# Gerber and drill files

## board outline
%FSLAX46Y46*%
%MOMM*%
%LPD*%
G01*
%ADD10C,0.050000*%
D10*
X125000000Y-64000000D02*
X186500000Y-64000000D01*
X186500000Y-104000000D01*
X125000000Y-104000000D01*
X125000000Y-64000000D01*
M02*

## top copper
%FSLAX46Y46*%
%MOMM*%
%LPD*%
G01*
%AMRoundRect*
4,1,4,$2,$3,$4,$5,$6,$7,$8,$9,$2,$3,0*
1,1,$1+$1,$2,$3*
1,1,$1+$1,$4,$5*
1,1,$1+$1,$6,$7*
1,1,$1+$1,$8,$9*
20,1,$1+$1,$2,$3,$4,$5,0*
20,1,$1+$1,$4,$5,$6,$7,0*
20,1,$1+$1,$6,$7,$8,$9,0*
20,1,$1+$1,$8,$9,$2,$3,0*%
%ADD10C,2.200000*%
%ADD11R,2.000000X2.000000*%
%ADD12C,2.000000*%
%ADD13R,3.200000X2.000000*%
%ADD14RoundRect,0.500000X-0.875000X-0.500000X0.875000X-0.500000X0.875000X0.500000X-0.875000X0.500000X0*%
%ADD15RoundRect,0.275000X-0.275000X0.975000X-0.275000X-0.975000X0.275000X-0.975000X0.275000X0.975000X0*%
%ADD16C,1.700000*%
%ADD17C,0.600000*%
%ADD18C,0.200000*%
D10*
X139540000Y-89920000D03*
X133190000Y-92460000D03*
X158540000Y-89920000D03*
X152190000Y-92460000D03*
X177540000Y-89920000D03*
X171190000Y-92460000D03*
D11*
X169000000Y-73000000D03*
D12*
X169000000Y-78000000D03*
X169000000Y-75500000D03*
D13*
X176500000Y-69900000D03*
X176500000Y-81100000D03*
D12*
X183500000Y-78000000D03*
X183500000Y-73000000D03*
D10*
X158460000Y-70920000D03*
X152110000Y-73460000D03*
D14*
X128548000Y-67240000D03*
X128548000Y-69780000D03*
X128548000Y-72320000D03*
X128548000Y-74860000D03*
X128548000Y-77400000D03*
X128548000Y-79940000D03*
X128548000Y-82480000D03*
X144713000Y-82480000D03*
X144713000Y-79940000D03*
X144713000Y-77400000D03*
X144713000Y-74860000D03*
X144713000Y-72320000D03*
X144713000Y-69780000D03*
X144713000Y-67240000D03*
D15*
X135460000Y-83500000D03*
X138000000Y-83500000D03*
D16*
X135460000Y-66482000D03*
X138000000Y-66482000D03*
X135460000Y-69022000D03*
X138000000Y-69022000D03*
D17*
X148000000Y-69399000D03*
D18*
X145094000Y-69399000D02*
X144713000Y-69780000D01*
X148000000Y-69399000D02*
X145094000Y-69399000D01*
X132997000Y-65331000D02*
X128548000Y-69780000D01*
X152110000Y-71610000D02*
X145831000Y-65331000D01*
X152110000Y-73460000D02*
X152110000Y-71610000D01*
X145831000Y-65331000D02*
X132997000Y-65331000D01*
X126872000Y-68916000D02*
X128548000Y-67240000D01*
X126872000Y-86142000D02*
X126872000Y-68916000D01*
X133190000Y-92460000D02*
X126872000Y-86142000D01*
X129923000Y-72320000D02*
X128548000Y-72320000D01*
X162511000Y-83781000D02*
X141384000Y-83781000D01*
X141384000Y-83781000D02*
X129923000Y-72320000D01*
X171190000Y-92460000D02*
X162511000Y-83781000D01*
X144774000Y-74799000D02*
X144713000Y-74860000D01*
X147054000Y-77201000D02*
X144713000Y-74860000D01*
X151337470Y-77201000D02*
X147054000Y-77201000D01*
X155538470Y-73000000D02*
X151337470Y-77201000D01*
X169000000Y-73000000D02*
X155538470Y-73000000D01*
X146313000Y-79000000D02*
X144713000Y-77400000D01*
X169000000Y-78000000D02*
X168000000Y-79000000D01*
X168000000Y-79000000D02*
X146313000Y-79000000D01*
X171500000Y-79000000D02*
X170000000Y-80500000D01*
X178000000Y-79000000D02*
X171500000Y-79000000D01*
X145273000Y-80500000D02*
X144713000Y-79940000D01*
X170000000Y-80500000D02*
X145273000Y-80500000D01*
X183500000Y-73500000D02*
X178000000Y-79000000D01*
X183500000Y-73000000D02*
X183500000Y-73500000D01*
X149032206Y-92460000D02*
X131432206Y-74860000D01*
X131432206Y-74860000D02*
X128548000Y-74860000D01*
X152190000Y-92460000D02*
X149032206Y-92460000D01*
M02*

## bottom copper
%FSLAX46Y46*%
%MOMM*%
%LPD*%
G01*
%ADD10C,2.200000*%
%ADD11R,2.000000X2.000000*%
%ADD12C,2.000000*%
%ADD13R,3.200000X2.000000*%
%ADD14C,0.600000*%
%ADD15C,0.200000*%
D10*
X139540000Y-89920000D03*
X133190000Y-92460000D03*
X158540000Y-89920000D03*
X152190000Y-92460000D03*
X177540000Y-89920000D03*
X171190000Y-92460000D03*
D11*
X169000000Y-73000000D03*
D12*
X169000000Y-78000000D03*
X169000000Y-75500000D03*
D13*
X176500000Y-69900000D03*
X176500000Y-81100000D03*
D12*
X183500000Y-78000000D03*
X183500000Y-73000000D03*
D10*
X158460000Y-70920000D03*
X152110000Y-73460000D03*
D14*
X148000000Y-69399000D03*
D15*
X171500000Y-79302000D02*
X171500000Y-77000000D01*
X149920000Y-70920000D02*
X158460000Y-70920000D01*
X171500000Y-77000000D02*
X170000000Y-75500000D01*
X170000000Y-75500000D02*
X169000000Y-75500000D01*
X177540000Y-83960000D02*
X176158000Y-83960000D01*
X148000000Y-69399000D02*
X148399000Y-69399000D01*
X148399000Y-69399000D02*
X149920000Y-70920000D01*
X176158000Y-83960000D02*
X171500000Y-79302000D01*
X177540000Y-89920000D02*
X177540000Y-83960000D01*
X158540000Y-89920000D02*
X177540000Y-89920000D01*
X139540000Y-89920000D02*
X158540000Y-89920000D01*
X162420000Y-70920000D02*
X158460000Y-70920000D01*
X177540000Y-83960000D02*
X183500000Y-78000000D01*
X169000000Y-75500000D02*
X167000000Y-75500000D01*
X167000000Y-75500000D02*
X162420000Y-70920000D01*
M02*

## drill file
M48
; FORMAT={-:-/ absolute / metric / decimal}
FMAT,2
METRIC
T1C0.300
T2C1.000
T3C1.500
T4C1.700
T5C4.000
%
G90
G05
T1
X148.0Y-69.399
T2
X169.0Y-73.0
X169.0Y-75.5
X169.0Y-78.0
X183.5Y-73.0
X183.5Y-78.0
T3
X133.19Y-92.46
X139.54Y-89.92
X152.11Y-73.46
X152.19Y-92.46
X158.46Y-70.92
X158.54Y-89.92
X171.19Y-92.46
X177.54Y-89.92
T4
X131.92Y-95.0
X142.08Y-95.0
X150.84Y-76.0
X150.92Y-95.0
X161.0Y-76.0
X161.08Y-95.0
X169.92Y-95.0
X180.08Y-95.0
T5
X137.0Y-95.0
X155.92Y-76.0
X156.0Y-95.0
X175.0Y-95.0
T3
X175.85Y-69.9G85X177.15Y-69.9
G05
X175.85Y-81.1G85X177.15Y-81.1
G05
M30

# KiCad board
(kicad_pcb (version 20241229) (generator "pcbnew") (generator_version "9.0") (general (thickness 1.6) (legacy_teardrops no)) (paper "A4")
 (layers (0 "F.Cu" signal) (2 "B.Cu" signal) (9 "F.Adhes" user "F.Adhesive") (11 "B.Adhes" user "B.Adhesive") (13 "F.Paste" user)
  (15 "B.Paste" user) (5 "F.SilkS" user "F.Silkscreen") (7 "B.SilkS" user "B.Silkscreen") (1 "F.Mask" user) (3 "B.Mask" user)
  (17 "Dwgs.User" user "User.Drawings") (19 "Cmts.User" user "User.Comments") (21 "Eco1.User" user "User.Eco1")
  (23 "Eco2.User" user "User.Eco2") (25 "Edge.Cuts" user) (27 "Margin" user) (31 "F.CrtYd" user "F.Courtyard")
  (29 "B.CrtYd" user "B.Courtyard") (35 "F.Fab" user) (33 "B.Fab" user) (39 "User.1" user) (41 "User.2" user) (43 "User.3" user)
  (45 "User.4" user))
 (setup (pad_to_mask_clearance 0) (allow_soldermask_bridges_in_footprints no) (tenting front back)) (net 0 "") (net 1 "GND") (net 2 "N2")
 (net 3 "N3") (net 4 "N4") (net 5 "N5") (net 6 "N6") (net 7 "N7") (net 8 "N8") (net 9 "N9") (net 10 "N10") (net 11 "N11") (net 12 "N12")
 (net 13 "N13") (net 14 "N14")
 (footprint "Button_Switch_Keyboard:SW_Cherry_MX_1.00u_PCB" (layer "F.Cu") (at 139.54 89.92)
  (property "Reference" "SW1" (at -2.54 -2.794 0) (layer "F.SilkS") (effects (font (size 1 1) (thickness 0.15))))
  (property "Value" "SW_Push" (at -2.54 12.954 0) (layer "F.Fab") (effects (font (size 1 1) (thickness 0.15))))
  (pad "" np_thru_hole circle (at -7.62 5.08) (size 1.7 1.7) (drill 1.7) (layers "*.Cu" "*.Mask"))
  (pad "" np_thru_hole circle (at -2.54 5.08) (size 4 4) (drill 4) (layers "*.Cu" "*.Mask"))
  (pad "" np_thru_hole circle (at 2.54 5.08) (size 1.7 1.7) (drill 1.7) (layers "*.Cu" "*.Mask"))
  (pad "1" thru_hole circle (at 0 0) (size 2.2 2.2) (drill 1.5) (layers "*.Cu" "*.Mask") (remove_unused_layers no) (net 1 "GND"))
  (pad "2" thru_hole circle (at -6.35 2.54) (size 2.2 2.2) (drill 1.5) (layers "*.Cu" "*.Mask") (remove_unused_layers no) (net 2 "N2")))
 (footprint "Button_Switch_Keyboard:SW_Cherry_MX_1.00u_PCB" (layer "F.Cu") (at 158.54 89.92)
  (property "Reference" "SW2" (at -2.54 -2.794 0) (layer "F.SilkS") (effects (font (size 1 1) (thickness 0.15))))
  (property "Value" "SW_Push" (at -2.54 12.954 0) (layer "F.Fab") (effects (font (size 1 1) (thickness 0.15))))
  (pad "" np_thru_hole circle (at -7.62 5.08) (size 1.7 1.7) (drill 1.7) (layers "*.Cu" "*.Mask"))
  (pad "" np_thru_hole circle (at -2.54 5.08) (size 4 4) (drill 4) (layers "*.Cu" "*.Mask"))
  (pad "" np_thru_hole circle (at 2.54 5.08) (size 1.7 1.7) (drill 1.7) (layers "*.Cu" "*.Mask"))
  (pad "1" thru_hole circle (at 0 0) (size 2.2 2.2) (drill 1.5) (layers "*.Cu" "*.Mask") (remove_unused_layers no) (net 1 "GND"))
  (pad "2" thru_hole circle (at -6.35 2.54) (size 2.2 2.2) (drill 1.5) (layers "*.Cu" "*.Mask") (remove_unused_layers no) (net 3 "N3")))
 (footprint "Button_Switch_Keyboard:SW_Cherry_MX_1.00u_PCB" (layer "F.Cu") (at 177.54 89.92)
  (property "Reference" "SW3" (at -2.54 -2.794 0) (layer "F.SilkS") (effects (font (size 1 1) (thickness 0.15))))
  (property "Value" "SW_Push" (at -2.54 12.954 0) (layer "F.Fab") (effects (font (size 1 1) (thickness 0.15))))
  (pad "" np_thru_hole circle (at -7.62 5.08) (size 1.7 1.7) (drill 1.7) (layers "*.Cu" "*.Mask"))
  (pad "" np_thru_hole circle (at -2.54 5.08) (size 4 4) (drill 4) (layers "*.Cu" "*.Mask"))
  (pad "" np_thru_hole circle (at 2.54 5.08) (size 1.7 1.7) (drill 1.7) (layers "*.Cu" "*.Mask"))
  (pad "1" thru_hole circle (at 0 0) (size 2.2 2.2) (drill 1.5) (layers "*.Cu" "*.Mask") (remove_unused_layers no) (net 1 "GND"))
  (pad "2" thru_hole circle (at -6.35 2.54) (size 2.2 2.2) (drill 1.5) (layers "*.Cu" "*.Mask") (remove_unused_layers no) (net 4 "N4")))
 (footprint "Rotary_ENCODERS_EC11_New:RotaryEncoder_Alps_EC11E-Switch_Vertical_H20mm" (layer "F.Cu") (at 169 73)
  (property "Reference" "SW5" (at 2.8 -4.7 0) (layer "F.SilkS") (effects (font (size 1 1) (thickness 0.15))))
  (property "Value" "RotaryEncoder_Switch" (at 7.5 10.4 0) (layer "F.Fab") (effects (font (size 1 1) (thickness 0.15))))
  (pad "A" thru_hole rect (at 0 0) (size 2 2) (drill 1) (layers "*.Cu" "*.Mask") (remove_unused_layers no) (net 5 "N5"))
  (pad "B" thru_hole circle (at 0 5) (size 2 2) (drill 1) (layers "*.Cu" "*.Mask") (remove_unused_layers no) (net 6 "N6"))
  (pad "C" thru_hole circle (at 0 2.5) (size 2 2) (drill 1) (layers "*.Cu" "*.Mask") (remove_unused_layers no) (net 1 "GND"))
  (pad "MP" thru_hole rect (at 7.5 -3.1) (size 3.2 2) (drill oval 2.8 1.5) (layers "*.Cu" "*.Mask") (remove_unused_layers no))
  (pad "MP" thru_hole rect (at 7.5 8.1) (size 3.2 2) (drill oval 2.8 1.5) (layers "*.Cu" "*.Mask") (remove_unused_layers no))
  (pad "S1" thru_hole circle (at 14.5 5) (size 2 2) (drill 1) (layers "*.Cu" "*.Mask") (remove_unused_layers no) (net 1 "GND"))
  (pad "S2" thru_hole circle (at 14.5 0) (size 2 2) (drill 1) (layers "*.Cu" "*.Mask") (remove_unused_layers no) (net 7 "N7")))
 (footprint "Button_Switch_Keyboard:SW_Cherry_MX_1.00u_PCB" (layer "F.Cu") (at 158.46 70.92)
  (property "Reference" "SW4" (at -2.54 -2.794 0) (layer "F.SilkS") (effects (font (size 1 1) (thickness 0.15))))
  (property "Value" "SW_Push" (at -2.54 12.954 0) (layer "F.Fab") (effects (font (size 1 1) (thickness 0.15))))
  (pad "" np_thru_hole circle (at -7.62 5.08) (size 1.7 1.7) (drill 1.7) (layers "*.Cu" "*.Mask"))
  (pad "" np_thru_hole circle (at -2.54 5.08) (size 4 4) (drill 4) (layers "*.Cu" "*.Mask"))
  (pad "" np_thru_hole circle (at 2.54 5.08) (size 1.7 1.7) (drill 1.7) (layers "*.Cu" "*.Mask"))
  (pad "1" thru_hole circle (at 0 0) (size 2.2 2.2) (drill 1.5) (layers "*.Cu" "*.Mask") (remove_unused_layers no) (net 1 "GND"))
  (pad "2" thru_hole circle (at -6.35 2.54) (size 2.2 2.2) (drill 1.5) (layers "*.Cu" "*.Mask") (remove_unused_layers no) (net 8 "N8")))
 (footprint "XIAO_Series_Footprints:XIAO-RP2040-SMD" (layer "F.Cu") (at 127.713 85.36)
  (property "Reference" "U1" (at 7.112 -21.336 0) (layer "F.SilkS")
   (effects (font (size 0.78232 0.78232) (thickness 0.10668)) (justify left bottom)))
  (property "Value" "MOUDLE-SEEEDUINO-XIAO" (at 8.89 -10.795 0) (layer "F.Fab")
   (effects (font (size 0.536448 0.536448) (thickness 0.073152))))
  (pad "1" smd roundrect (at 0.835 -18.12) (size 2.75 2) (layers "F.Cu" "F.Mask" "F.Paste") (roundrect_rratio 0.25) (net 2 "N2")
   (solder_mask_margin 0.0508) (thermal_bridge_angle 45))
  (pad "2" smd roundrect (at 0.835 -15.58) (size 2.75 2) (layers "F.Cu" "F.Mask" "F.Paste") (roundrect_rratio 0.25) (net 8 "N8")
   (solder_mask_margin 0.0508) (thermal_bridge_angle 45))
  (pad "3" smd roundrect (at 0.835 -13.04) (size 2.75 2) (layers "F.Cu" "F.Mask" "F.Paste") (roundrect_rratio 0.25) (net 4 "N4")
   (solder_mask_margin 0.0508) (thermal_bridge_angle 45))
  (pad "4" smd roundrect (at 0.835 -10.5) (size 2.75 2) (layers "F.Cu" "F.Mask" "F.Paste") (roundrect_rratio 0.25) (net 3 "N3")
   (solder_mask_margin 0.0508) (thermal_bridge_angle 45))
  (pad "5" smd roundrect (at 0.835 -7.96) (size 2.75 2) (layers "F.Cu" "F.Mask" "F.Paste") (roundrect_rratio 0.25) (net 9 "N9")
   (solder_mask_margin 0.0508) (thermal_bridge_angle 45))
  (pad "6" smd roundrect (at 0.835 -5.42) (size 2.75 2) (layers "F.Cu" "F.Mask" "F.Paste") (roundrect_rratio 0.25) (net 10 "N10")
   (solder_mask_margin 0.0508) (thermal_bridge_angle 45))
  (pad "7" smd roundrect (at 0.835 -2.88) (size 2.75 2) (layers "F.Cu" "F.Mask" "F.Paste") (roundrect_rratio 0.25) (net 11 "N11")
   (solder_mask_margin 0.0508) (thermal_bridge_angle 45))
  (pad "8" smd roundrect (at 17 -2.88) (size 2.75 2) (layers "F.Cu" "F.Mask" "F.Paste") (roundrect_rratio 0.25) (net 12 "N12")
   (solder_mask_margin 0.0508) (thermal_bridge_angle 45))
  (pad "9" smd roundrect (at 17 -5.42) (size 2.75 2) (layers "F.Cu" "F.Mask" "F.Paste") (roundrect_rratio 0.25) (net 7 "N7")
   (solder_mask_margin 0.0508) (thermal_bridge_angle 45))
  (pad "10" smd roundrect (at 17 -7.96) (size 2.75 2) (layers "F.Cu" "F.Mask" "F.Paste") (roundrect_rratio 0.25) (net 6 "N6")
   (solder_mask_margin 0.0508) (thermal_bridge_angle 45))
  (pad "11" smd roundrect (at 17 -10.5) (size 2.75 2) (layers "F.Cu" "F.Mask" "F.Paste") (roundrect_rratio 0.25) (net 5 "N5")
   (solder_mask_margin 0.0508) (thermal_bridge_angle 45))
  (pad "12" smd roundrect (at 17 -13.04) (size 2.75 2) (layers "F.Cu" "F.Mask" "F.Paste") (roundrect_rratio 0.25) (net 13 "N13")
   (solder_mask_margin 0.0508) (thermal_bridge_angle 45))
  (pad "13" smd roundrect (at 17 -15.58) (size 2.75 2) (layers "F.Cu" "F.Mask" "F.Paste") (roundrect_rratio 0.25) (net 1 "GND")
   (solder_mask_margin 0.0508) (thermal_bridge_angle 45))
  (pad "14" smd roundrect (at 17 -18.12) (size 2.75 2) (layers "F.Cu" "F.Mask" "F.Paste") (roundrect_rratio 0.25) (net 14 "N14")
   (solder_mask_margin 0.0508) (thermal_bridge_angle 45))
  (pad "15" smd roundrect (at 7.747 -1.86 270) (size 2.5 1.1) (layers "F.Cu" "F.Mask" "F.Paste") (roundrect_rratio 0.25)
   (thermal_bridge_angle 45))
  (pad "16" smd roundrect (at 10.287 -1.86 270) (size 2.5 1.1) (layers "F.Cu" "F.Mask" "F.Paste") (roundrect_rratio 0.25)
   (thermal_bridge_angle 45))
  (pad "17" smd circle (at 7.747 -18.878) (size 1.7 1.7) (layers "F.Cu" "F.Mask" "F.Paste"))
  (pad "18" smd circle (at 10.287 -18.878) (size 1.7 1.7) (layers "F.Cu" "F.Mask" "F.Paste"))
  (pad "19" smd circle (at 7.747 -16.338) (size 1.7 1.7) (layers "F.Cu" "F.Mask" "F.Paste"))
  (pad "20" smd circle (at 10.287 -16.338) (size 1.7 1.7) (layers "F.Cu" "F.Mask" "F.Paste")))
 (gr_rect (start 125 64) (end 186.5 104) (stroke (width 0.05) (type default)) (fill no) (layer "Edge.Cuts"))
 (segment (start 145.094 69.399) (end 144.713 69.78) (width 0.2) (layer "F.Cu") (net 1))
 (segment (start 148 69.399) (end 145.094 69.399) (width 0.2) (layer "F.Cu") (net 1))
 (via (at 148 69.399) (size 0.6) (drill 0.3) (layers "F.Cu" "B.Cu") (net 1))
 (segment (start 171.5 79.302) (end 171.5 77) (width 0.2) (layer "B.Cu") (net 1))
 (segment (start 149.92 70.92) (end 158.46 70.92) (width 0.2) (layer "B.Cu") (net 1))
 (segment (start 171.5 77) (end 170 75.5) (width 0.2) (layer "B.Cu") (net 1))
 (segment (start 170 75.5) (end 169 75.5) (width 0.2) (layer "B.Cu") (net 1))
 (segment (start 177.54 83.96) (end 176.158 83.96) (width 0.2) (layer "B.Cu") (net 1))
 (segment (start 148 69.399) (end 148.399 69.399) (width 0.2) (layer "B.Cu") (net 1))
 (segment (start 148.399 69.399) (end 149.92 70.92) (width 0.2) (layer "B.Cu") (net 1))
 (segment (start 176.158 83.96) (end 171.5 79.302) (width 0.2) (layer "B.Cu") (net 1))
 (segment (start 177.54 89.92) (end 177.54 83.96) (width 0.2) (layer "B.Cu") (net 1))
 (segment (start 158.54 89.92) (end 177.54 89.92) (width 0.2) (layer "B.Cu") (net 1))
 (segment (start 139.54 89.92) (end 158.54 89.92) (width 0.2) (layer "B.Cu") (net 1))
 (segment (start 162.42 70.92) (end 158.46 70.92) (width 0.2) (layer "B.Cu") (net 1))
 (segment (start 177.54 83.96) (end 183.5 78) (width 0.2) (layer "B.Cu") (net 1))
 (segment (start 169 75.5) (end 167 75.5) (width 0.2) (layer "B.Cu") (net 1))
 (segment (start 167 75.5) (end 162.42 70.92) (width 0.2) (layer "B.Cu") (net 1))
 (segment (start 132.997 65.331) (end 128.548 69.78) (width 0.2) (layer "F.Cu") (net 8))
 (segment (start 152.11 71.61) (end 145.831 65.331) (width 0.2) (layer "F.Cu") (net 8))
 (segment (start 152.11 73.46) (end 152.11 71.61) (width 0.2) (layer "F.Cu") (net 8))
 (segment (start 145.831 65.331) (end 132.997 65.331) (width 0.2) (layer "F.Cu") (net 8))
 (segment (start 126.872 68.916) (end 128.548 67.24) (width 0.2) (layer "F.Cu") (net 2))
 (segment (start 126.872 86.142) (end 126.872 68.916) (width 0.2) (layer "F.Cu") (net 2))
 (segment (start 133.19 92.46) (end 126.872 86.142) (width 0.2) (layer "F.Cu") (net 2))
 (segment (start 129.923 72.32) (end 128.548 72.32) (width 0.2) (layer "F.Cu") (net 4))
 (segment (start 162.511 83.781) (end 141.384 83.781) (width 0.2) (layer "F.Cu") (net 4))
 (segment (start 141.384 83.781) (end 129.923 72.32) (width 0.2) (layer "F.Cu") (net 4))
 (segment (start 171.19 92.46) (end 162.511 83.781) (width 0.2) (layer "F.Cu") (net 4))
 (segment (start 144.774 74.799) (end 144.713 74.86) (width 0.2) (layer "F.Cu") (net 5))
 (segment (start 147.054 77.201) (end 144.713 74.86) (width 0.2) (layer "F.Cu") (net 5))
 (segment (start 151.33747 77.201) (end 147.054 77.201) (width 0.2) (layer "F.Cu") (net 5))
 (segment (start 155.53847 73) (end 151.33747 77.201) (width 0.2) (layer "F.Cu") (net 5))
 (segment (start 169 73) (end 155.53847 73) (width 0.2) (layer "F.Cu") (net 5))
 (segment (start 146.313 79) (end 144.713 77.4) (width 0.2) (layer "F.Cu") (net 6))
 (segment (start 169 78) (end 168 79) (width 0.2) (layer "F.Cu") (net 6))
 (segment (start 168 79) (end 146.313 79) (width 0.2) (layer "F.Cu") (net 6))
 (segment (start 171.5 79) (end 170 80.5) (width 0.2) (layer "F.Cu") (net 7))
 (segment (start 178 79) (end 171.5 79) (width 0.2) (layer "F.Cu") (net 7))
 (segment (start 145.273 80.5) (end 144.713 79.94) (width 0.2) (layer "F.Cu") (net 7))
 (segment (start 170 80.5) (end 145.273 80.5) (width 0.2) (layer "F.Cu") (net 7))
 (segment (start 183.5 73.5) (end 178 79) (width 0.2) (layer "F.Cu") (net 7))
 (segment (start 183.5 73) (end 183.5 73.5) (width 0.2) (layer "F.Cu") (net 7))
 (segment (start 149.032206 92.46) (end 131.432206 74.86) (width 0.2) (layer "F.Cu") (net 3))
 (segment (start 131.432206 74.86) (end 128.548 74.86) (width 0.2) (layer "F.Cu") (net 3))
 (segment (start 152.19 92.46) (end 149.032206 92.46) (width 0.2) (layer "F.Cu") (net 3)))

